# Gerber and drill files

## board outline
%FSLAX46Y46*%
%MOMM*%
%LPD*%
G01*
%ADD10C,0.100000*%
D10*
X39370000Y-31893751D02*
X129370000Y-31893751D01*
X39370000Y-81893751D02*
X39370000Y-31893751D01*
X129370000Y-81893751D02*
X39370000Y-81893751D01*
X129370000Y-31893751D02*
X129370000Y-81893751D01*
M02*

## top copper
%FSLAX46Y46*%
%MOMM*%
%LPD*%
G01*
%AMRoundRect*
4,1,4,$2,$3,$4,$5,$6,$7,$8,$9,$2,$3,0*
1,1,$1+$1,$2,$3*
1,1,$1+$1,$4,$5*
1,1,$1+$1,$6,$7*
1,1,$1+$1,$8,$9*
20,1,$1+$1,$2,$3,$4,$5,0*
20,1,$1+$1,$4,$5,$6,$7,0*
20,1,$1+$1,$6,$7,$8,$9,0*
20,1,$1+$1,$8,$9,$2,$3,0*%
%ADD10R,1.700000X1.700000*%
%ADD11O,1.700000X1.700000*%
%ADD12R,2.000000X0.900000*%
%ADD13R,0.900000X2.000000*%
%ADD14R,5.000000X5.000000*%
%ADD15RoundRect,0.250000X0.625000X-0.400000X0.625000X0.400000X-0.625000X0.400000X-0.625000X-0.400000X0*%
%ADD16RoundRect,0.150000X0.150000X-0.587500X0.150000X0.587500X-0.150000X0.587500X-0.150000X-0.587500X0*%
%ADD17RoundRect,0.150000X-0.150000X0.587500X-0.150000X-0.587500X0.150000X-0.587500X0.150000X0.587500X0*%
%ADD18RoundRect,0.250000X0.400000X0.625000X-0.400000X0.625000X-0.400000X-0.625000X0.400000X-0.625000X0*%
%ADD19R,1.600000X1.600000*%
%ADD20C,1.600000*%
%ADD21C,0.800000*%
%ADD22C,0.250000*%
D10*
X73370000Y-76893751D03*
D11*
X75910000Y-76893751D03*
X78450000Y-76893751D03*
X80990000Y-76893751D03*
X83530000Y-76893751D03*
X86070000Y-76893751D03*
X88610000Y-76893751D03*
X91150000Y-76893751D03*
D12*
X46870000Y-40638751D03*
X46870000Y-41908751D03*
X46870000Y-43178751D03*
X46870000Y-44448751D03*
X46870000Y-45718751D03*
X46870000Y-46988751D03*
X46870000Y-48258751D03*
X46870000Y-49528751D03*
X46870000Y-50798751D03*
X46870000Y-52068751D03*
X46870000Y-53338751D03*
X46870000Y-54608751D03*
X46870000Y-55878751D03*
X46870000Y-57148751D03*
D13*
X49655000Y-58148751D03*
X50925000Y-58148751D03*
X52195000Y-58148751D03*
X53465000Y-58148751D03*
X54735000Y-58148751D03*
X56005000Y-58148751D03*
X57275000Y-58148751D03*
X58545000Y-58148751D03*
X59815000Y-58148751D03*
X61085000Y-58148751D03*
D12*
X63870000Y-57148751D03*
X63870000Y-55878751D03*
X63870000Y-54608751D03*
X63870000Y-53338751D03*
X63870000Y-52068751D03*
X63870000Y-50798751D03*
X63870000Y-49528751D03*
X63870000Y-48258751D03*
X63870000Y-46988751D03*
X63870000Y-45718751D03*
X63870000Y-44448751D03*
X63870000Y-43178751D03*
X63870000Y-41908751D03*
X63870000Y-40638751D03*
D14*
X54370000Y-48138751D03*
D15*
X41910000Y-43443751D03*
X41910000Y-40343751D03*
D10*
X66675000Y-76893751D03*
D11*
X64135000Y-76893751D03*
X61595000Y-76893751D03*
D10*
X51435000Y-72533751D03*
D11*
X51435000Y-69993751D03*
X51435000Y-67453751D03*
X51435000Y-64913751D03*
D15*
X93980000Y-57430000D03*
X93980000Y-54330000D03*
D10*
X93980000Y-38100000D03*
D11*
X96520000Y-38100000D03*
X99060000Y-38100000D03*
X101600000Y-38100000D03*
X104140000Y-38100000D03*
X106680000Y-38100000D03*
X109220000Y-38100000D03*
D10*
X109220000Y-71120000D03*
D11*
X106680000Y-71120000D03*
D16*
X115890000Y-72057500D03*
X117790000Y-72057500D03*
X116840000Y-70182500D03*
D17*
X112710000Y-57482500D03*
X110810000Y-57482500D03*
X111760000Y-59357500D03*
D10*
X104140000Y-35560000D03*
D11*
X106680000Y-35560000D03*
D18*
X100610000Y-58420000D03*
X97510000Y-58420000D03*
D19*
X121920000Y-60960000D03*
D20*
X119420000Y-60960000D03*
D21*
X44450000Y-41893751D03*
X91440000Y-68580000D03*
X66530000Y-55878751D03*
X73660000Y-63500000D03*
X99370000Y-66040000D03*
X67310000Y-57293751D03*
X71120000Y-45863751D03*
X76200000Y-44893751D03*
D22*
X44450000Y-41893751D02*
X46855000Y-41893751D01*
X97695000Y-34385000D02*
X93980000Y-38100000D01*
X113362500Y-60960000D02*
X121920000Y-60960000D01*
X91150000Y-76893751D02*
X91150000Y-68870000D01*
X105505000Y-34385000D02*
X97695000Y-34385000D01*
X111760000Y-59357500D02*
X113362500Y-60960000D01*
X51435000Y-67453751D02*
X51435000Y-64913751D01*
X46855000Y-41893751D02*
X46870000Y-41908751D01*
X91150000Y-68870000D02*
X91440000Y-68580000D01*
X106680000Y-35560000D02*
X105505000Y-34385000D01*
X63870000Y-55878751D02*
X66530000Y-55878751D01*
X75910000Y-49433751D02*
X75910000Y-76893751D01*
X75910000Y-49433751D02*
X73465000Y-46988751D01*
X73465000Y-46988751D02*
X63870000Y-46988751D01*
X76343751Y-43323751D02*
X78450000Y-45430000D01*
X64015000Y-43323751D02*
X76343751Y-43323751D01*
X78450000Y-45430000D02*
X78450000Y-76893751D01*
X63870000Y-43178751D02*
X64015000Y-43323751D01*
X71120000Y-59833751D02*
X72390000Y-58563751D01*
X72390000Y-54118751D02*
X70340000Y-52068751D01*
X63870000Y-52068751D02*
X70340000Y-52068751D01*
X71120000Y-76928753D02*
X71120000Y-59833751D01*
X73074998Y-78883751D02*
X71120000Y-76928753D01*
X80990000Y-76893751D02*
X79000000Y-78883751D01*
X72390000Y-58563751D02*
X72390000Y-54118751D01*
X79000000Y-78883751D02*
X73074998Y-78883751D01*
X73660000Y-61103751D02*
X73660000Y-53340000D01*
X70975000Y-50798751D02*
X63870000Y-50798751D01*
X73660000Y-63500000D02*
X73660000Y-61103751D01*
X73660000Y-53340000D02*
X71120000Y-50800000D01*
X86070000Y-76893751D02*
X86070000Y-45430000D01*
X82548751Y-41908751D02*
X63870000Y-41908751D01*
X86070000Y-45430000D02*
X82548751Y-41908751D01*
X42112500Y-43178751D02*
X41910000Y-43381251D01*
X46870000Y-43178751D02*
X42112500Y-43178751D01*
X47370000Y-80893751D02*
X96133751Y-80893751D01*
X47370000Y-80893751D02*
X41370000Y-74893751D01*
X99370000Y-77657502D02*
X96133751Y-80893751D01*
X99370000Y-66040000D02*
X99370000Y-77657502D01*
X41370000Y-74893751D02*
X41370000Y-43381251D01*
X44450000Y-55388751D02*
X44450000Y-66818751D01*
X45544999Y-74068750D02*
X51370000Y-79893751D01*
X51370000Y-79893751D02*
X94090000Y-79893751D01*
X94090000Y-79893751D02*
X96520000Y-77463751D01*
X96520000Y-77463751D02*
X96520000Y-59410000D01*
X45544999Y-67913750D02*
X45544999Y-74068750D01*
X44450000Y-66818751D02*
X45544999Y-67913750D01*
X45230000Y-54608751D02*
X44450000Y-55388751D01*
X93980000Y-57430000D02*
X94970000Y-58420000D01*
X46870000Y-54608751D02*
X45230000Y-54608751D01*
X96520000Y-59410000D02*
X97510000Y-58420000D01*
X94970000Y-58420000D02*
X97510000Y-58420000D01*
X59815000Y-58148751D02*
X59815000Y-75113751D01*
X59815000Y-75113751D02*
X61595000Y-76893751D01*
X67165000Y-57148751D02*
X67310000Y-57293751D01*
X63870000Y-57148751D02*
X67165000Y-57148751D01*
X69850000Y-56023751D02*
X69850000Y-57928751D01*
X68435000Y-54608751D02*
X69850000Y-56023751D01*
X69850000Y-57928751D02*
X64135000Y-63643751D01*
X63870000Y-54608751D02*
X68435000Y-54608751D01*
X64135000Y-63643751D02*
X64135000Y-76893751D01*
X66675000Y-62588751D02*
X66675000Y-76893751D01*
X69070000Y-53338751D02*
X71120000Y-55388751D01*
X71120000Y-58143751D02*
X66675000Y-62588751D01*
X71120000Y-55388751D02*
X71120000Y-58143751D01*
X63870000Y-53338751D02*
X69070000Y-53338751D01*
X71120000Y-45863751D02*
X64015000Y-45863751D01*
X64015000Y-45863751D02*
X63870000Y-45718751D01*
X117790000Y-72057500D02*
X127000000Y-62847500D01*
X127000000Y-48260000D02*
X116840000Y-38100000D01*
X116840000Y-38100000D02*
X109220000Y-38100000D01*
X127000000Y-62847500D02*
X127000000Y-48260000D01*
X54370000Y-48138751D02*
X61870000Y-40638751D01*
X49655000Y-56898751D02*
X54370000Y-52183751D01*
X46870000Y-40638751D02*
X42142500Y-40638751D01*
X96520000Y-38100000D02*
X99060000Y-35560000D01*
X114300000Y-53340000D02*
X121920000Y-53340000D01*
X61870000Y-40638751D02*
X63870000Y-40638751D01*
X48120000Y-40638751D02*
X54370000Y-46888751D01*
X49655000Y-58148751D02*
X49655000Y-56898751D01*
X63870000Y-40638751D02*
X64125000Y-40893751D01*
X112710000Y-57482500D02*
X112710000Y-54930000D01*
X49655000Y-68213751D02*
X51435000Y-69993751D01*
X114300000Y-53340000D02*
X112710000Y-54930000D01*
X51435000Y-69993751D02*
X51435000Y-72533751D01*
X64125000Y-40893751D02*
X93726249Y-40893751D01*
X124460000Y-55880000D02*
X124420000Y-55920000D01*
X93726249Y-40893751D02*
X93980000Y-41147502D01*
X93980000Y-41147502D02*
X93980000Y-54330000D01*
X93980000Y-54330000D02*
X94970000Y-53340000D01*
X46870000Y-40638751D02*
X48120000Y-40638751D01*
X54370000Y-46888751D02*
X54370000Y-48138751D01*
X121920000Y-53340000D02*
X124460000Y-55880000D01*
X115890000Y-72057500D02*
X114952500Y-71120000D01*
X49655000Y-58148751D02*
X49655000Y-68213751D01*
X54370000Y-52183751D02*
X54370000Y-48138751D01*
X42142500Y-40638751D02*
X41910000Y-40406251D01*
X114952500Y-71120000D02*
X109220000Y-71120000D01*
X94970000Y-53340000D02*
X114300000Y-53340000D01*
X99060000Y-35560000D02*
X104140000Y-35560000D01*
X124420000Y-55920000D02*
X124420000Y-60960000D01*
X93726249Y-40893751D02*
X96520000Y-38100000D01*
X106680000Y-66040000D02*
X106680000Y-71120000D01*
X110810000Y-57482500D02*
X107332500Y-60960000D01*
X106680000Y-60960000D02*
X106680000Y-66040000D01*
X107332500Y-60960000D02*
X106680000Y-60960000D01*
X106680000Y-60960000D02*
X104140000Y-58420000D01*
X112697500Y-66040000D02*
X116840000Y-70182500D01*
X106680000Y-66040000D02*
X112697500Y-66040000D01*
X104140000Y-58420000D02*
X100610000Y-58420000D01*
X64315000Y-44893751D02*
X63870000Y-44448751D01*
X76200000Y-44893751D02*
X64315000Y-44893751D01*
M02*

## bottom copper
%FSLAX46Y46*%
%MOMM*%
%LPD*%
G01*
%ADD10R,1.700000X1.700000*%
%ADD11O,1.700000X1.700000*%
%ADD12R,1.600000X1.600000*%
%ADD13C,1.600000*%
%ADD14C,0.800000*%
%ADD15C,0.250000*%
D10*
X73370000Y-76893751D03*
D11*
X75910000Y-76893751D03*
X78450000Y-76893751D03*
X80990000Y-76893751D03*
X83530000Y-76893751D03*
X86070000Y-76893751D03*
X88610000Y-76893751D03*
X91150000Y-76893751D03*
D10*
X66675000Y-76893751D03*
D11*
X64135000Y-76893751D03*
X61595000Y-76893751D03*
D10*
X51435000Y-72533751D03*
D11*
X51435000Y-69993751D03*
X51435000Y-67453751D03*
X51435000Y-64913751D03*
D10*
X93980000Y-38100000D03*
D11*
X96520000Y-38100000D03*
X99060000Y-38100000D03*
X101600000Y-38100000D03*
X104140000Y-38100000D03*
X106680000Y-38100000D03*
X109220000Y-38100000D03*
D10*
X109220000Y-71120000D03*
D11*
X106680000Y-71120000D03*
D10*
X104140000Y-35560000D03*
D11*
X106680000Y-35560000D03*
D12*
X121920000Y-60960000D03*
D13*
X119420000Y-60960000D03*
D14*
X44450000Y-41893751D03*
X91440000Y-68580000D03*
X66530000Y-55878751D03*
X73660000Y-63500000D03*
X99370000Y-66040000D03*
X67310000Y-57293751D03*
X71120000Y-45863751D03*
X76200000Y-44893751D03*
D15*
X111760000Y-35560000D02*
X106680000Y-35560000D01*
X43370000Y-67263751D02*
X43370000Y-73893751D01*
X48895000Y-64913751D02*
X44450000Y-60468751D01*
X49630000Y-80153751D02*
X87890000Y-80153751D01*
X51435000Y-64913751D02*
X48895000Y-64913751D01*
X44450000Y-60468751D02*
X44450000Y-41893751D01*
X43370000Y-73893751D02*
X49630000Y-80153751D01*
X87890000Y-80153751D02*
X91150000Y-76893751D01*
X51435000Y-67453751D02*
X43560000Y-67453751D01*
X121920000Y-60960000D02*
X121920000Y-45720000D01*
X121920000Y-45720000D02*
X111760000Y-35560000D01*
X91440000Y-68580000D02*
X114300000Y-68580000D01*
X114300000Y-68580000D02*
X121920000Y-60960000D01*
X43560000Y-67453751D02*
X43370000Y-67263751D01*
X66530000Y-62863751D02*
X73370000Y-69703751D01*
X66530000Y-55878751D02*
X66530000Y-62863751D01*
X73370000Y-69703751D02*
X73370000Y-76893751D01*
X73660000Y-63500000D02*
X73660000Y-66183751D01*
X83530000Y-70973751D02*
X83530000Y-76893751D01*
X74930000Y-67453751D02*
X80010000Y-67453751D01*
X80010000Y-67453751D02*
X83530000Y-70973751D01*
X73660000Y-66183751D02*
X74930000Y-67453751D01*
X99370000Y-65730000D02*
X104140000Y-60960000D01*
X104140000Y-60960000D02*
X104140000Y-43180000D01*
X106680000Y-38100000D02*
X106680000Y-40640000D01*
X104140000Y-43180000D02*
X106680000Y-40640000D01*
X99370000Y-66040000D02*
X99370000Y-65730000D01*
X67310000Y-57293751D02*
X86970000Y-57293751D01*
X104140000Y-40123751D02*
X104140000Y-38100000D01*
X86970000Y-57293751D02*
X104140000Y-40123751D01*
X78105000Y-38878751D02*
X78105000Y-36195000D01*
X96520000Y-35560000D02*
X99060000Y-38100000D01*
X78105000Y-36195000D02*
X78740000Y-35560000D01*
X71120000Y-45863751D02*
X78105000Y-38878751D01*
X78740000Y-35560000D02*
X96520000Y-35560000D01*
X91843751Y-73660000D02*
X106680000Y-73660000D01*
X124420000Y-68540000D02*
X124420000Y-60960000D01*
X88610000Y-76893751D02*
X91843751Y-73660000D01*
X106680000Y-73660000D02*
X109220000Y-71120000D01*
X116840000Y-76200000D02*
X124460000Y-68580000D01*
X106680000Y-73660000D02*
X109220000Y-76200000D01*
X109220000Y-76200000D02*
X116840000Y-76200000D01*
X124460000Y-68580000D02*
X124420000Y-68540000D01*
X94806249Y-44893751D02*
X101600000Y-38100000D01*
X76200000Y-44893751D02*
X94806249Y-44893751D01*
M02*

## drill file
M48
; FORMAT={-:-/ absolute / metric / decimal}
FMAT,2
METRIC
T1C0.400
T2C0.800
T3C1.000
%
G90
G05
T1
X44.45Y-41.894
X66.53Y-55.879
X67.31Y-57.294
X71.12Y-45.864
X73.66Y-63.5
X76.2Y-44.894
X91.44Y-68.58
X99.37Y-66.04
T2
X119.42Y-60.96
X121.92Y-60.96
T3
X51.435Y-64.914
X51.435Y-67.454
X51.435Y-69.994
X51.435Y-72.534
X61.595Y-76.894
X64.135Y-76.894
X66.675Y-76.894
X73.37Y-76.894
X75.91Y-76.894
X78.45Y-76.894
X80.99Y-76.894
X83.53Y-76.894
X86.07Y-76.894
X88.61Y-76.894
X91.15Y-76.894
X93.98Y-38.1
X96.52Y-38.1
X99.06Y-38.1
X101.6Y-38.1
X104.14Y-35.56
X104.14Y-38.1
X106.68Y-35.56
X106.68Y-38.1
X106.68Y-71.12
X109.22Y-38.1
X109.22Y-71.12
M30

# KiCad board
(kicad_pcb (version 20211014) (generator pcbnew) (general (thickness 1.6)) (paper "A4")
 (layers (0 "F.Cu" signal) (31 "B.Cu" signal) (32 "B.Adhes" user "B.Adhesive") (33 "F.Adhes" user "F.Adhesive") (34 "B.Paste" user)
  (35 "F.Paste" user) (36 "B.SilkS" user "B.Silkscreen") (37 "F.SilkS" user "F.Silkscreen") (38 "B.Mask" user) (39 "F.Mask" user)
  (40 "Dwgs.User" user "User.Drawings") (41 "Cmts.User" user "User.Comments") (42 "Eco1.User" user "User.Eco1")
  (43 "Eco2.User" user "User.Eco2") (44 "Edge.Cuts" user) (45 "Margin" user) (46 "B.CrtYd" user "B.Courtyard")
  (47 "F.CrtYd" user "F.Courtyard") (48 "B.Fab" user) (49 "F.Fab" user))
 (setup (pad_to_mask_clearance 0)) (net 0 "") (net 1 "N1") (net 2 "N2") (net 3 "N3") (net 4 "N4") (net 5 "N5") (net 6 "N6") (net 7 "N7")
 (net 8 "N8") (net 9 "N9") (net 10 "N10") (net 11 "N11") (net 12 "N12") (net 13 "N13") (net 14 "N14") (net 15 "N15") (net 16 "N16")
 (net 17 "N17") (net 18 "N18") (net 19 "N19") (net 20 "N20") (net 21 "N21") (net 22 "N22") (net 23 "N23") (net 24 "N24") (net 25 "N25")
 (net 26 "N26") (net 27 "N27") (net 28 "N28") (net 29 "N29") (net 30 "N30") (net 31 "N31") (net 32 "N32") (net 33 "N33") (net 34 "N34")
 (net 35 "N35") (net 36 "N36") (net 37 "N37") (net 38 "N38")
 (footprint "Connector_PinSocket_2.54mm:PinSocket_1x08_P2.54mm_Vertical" (layer "F.Cu") (at 73.37 76.893751 90)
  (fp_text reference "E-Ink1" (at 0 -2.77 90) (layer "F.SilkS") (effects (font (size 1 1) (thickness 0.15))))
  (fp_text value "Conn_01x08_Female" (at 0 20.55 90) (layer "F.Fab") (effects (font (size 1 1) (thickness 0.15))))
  (pad "1" thru_hole rect locked (at 0 0 90) (size 1.7 1.7) (drill 1) (layers *.Cu *.Mask) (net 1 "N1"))
  (pad "2" thru_hole oval locked (at 0 2.54 90) (size 1.7 1.7) (drill 1) (layers *.Cu *.Mask) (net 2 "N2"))
  (pad "3" thru_hole oval locked (at 0 5.08 90) (size 1.7 1.7) (drill 1) (layers *.Cu *.Mask) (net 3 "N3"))
  (pad "4" thru_hole oval locked (at 0 7.62 90) (size 1.7 1.7) (drill 1) (layers *.Cu *.Mask) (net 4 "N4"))
  (pad "5" thru_hole oval locked (at 0 10.16 90) (size 1.7 1.7) (drill 1) (layers *.Cu *.Mask) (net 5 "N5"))
  (pad "6" thru_hole oval locked (at 0 12.7 90) (size 1.7 1.7) (drill 1) (layers *.Cu *.Mask) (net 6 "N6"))
  (pad "7" thru_hole oval locked (at 0 15.24 90) (size 1.7 1.7) (drill 1) (layers *.Cu *.Mask) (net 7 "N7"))
  (pad "8" thru_hole oval locked (at 0 17.78 90) (size 1.7 1.7) (drill 1) (layers *.Cu *.Mask) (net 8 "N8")))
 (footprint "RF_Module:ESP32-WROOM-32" (layer "F.Cu") (at 55.37 48.893751)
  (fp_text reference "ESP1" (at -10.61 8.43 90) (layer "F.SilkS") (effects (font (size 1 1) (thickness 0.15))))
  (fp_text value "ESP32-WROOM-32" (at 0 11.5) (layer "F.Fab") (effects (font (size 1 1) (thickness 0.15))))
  (pad "1" smd rect locked (at -8.5 -8.255) (size 2 0.9) (layers "F.Cu" "F.Paste" "F.Mask") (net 7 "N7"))
  (pad "2" smd rect locked (at -8.5 -6.985) (size 2 0.9) (layers "F.Cu" "F.Paste" "F.Mask") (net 8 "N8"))
  (pad "3" smd rect locked (at -8.5 -5.715) (size 2 0.9) (layers "F.Cu" "F.Paste" "F.Mask") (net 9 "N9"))
  (pad "4" smd rect locked (at -8.5 -4.445) (size 2 0.9) (layers "F.Cu" "F.Paste" "F.Mask") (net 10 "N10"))
  (pad "5" smd rect locked (at -8.5 -3.175) (size 2 0.9) (layers "F.Cu" "F.Paste" "F.Mask") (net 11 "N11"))
  (pad "6" smd rect locked (at -8.5 -1.905) (size 2 0.9) (layers "F.Cu" "F.Paste" "F.Mask") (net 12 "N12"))
  (pad "7" smd rect locked (at -8.5 -0.635) (size 2 0.9) (layers "F.Cu" "F.Paste" "F.Mask") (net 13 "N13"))
  (pad "8" smd rect locked (at -8.5 0.635) (size 2 0.9) (layers "F.Cu" "F.Paste" "F.Mask") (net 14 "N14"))
  (pad "9" smd rect locked (at -8.5 1.905) (size 2 0.9) (layers "F.Cu" "F.Paste" "F.Mask") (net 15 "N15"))
  (pad "10" smd rect locked (at -8.5 3.175) (size 2 0.9) (layers "F.Cu" "F.Paste" "F.Mask") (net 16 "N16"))
  (pad "11" smd rect locked (at -8.5 4.445) (size 2 0.9) (layers "F.Cu" "F.Paste" "F.Mask") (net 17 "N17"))
  (pad "12" smd rect locked (at -8.5 5.715) (size 2 0.9) (layers "F.Cu" "F.Paste" "F.Mask") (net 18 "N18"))
  (pad "13" smd rect locked (at -8.5 6.985) (size 2 0.9) (layers "F.Cu" "F.Paste" "F.Mask") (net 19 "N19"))
  (pad "14" smd rect locked (at -8.5 8.255) (size 2 0.9) (layers "F.Cu" "F.Paste" "F.Mask") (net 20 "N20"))
  (pad "15" smd rect locked (at -5.715 9.255 90) (size 2 0.9) (layers "F.Cu" "F.Paste" "F.Mask") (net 7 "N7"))
  (pad "16" smd rect locked (at -4.445 9.255 90) (size 2 0.9) (layers "F.Cu" "F.Paste" "F.Mask") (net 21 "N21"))
  (pad "17" smd rect locked (at -3.175 9.255 90) (size 2 0.9) (layers "F.Cu" "F.Paste" "F.Mask") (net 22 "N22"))
  (pad "18" smd rect locked (at -1.905 9.255 90) (size 2 0.9) (layers "F.Cu" "F.Paste" "F.Mask") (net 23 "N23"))
  (pad "19" smd rect locked (at -0.635 9.255 90) (size 2 0.9) (layers "F.Cu" "F.Paste" "F.Mask") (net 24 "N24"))
  (pad "20" smd rect locked (at 0.635 9.255 90) (size 2 0.9) (layers "F.Cu" "F.Paste" "F.Mask") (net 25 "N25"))
  (pad "21" smd rect locked (at 1.905 9.255 90) (size 2 0.9) (layers "F.Cu" "F.Paste" "F.Mask") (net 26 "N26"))
  (pad "22" smd rect locked (at 3.175 9.255 90) (size 2 0.9) (layers "F.Cu" "F.Paste" "F.Mask") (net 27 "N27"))
  (pad "23" smd rect locked (at 4.445 9.255 90) (size 2 0.9) (layers "F.Cu" "F.Paste" "F.Mask") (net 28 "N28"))
  (pad "24" smd rect locked (at 5.715 9.255 90) (size 2 0.9) (layers "F.Cu" "F.Paste" "F.Mask") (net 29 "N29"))
  (pad "25" smd rect locked (at 8.5 8.255) (size 2 0.9) (layers "F.Cu" "F.Paste" "F.Mask") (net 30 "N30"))
  (pad "26" smd rect locked (at 8.5 6.985) (size 2 0.9) (layers "F.Cu" "F.Paste" "F.Mask") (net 1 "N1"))
  (pad "27" smd rect locked (at 8.5 5.715) (size 2 0.9) (layers "F.Cu" "F.Paste" "F.Mask") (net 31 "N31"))
  (pad "28" smd rect locked (at 8.5 4.445) (size 2 0.9) (layers "F.Cu" "F.Paste" "F.Mask") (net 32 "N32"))
  (pad "29" smd rect locked (at 8.5 3.175) (size 2 0.9) (layers "F.Cu" "F.Paste" "F.Mask") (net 4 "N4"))
  (pad "30" smd rect locked (at 8.5 1.905) (size 2 0.9) (layers "F.Cu" "F.Paste" "F.Mask") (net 5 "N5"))
  (pad "31" smd rect locked (at 8.5 0.635) (size 2 0.9) (layers "F.Cu" "F.Paste" "F.Mask") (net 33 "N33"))
  (pad "32" smd rect locked (at 8.5 -0.635) (size 2 0.9) (layers "F.Cu" "F.Paste" "F.Mask") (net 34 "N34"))
  (pad "33" smd rect locked (at 8.5 -1.905) (size 2 0.9) (layers "F.Cu" "F.Paste" "F.Mask") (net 2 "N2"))
  (pad "34" smd rect locked (at 8.5 -3.175) (size 2 0.9) (layers "F.Cu" "F.Paste" "F.Mask") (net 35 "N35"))
  (pad "35" smd rect locked (at 8.5 -4.445) (size 2 0.9) (layers "F.Cu" "F.Paste" "F.Mask") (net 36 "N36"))
  (pad "36" smd rect locked (at 8.5 -5.715) (size 2 0.9) (layers "F.Cu" "F.Paste" "F.Mask") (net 3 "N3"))
  (pad "37" smd rect locked (at 8.5 -6.985) (size 2 0.9) (layers "F.Cu" "F.Paste" "F.Mask") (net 6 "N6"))
  (pad "38" smd rect locked (at 8.5 -8.255) (size 2 0.9) (layers "F.Cu" "F.Paste" "F.Mask") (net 7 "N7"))
  (pad "39" smd rect locked (at -1 -0.755) (size 5 5) (layers "F.Cu" "F.Paste" "F.Mask") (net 7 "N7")))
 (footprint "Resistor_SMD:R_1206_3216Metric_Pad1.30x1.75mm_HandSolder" (layer "F.Cu") (at 41.91 41.893751 90)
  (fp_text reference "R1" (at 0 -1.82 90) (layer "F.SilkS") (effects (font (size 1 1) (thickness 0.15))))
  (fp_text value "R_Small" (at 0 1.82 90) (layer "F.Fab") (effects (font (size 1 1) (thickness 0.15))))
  (pad "1" smd roundrect (at -1.55 0 90) (size 1.3 1.75) (layers "F.Cu" "F.Paste" "F.Mask") (roundrect_rratio 0.192308) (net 9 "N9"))
  (pad "2" smd roundrect (at 1.55 0 90) (size 1.3 1.75) (layers "F.Cu" "F.Paste" "F.Mask") (roundrect_rratio 0.192308) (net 7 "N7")))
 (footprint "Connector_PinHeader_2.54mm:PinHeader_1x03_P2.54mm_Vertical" (layer "F.Cu") (at 66.675 76.893751 -90)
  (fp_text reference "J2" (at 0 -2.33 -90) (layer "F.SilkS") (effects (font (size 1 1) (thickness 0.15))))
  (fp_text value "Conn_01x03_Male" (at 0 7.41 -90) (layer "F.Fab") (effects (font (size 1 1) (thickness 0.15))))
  (pad "1" thru_hole rect (at 0 0 270) (size 1.7 1.7) (drill 1) (layers *.Cu *.Mask) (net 32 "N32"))
  (pad "2" thru_hole oval (at 0 2.54 270) (size 1.7 1.7) (drill 1) (layers *.Cu *.Mask) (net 31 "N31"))
  (pad "3" thru_hole oval (at 0 5.08 270) (size 1.7 1.7) (drill 1) (layers *.Cu *.Mask) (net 28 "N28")))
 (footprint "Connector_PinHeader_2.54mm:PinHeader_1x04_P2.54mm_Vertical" (layer "F.Cu") (at 51.435 72.533751 180)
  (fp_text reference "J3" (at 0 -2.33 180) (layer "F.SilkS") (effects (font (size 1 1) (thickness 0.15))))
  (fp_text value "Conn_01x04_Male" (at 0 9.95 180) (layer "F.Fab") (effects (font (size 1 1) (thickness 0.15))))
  (pad "1" thru_hole rect (at 0 0 180) (size 1.7 1.7) (drill 1) (layers *.Cu *.Mask) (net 7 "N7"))
  (pad "2" thru_hole oval (at 0 2.54 180) (size 1.7 1.7) (drill 1) (layers *.Cu *.Mask) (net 7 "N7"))
  (pad "3" thru_hole oval (at 0 5.08 180) (size 1.7 1.7) (drill 1) (layers *.Cu *.Mask) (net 8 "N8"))
  (pad "4" thru_hole oval (at 0 7.62 180) (size 1.7 1.7) (drill 1) (layers *.Cu *.Mask) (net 8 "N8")))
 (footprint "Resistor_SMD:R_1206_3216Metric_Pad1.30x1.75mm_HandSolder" (layer "F.Cu") (at 93.98 55.88 90)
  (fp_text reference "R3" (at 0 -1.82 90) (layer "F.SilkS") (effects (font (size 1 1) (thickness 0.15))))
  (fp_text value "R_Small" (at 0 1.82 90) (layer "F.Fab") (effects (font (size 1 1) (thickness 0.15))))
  (pad "1" smd roundrect (at -1.55 0 90) (size 1.3 1.75) (layers "F.Cu" "F.Paste" "F.Mask") (roundrect_rratio 0.192308) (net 18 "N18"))
  (pad "2" smd roundrect (at 1.55 0 90) (size 1.3 1.75) (layers "F.Cu" "F.Paste" "F.Mask") (roundrect_rratio 0.192308) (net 7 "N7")))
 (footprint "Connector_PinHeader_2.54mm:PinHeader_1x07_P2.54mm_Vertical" (layer "F.Cu") (at 93.98 38.1 90)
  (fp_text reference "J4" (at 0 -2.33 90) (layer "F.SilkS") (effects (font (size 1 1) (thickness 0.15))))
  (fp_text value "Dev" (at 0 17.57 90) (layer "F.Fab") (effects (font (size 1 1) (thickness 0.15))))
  (pad "1" thru_hole rect (at 0 0 90) (size 1.7 1.7) (drill 1) (layers *.Cu *.Mask) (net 8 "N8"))
  (pad "2" thru_hole oval (at 0 2.54 90) (size 1.7 1.7) (drill 1) (layers *.Cu *.Mask) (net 7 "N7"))
  (pad "3" thru_hole oval (at 0 5.08 90) (size 1.7 1.7) (drill 1) (layers *.Cu *.Mask) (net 35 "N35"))
  (pad "4" thru_hole oval (at 0 7.62 90) (size 1.7 1.7) (drill 1) (layers *.Cu *.Mask) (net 36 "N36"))
  (pad "5" thru_hole oval (at 0 10.16 90) (size 1.7 1.7) (drill 1) (layers *.Cu *.Mask) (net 30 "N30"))
  (pad "6" thru_hole oval (at 0 12.7 90) (size 1.7 1.7) (drill 1) (layers *.Cu *.Mask) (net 9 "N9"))
  (pad "7" thru_hole oval (at 0 15.24 90) (size 1.7 1.7) (drill 1) (layers *.Cu *.Mask) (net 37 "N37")))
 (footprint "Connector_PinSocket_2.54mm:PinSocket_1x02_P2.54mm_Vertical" (layer "F.Cu") (at 109.22 71.12 -90)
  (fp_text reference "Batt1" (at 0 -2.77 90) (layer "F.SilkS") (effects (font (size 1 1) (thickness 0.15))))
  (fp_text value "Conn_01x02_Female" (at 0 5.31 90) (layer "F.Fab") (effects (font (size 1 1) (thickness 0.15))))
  (pad "1" thru_hole rect (at 0 0 270) (size 1.7 1.7) (drill 1) (layers *.Cu *.Mask) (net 7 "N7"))
  (pad "2" thru_hole oval (at 0 2.54 270) (size 1.7 1.7) (drill 1) (layers *.Cu *.Mask) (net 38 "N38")))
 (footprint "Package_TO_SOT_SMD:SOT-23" (layer "F.Cu") (at 116.84 71.12 90)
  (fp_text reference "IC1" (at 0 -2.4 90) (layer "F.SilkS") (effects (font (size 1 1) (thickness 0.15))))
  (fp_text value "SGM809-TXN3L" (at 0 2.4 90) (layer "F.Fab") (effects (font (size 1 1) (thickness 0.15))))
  (pad "1" smd roundrect (at -0.9375 -0.95 90) (size 1.475 0.6) (layers "F.Cu" "F.Paste" "F.Mask") (roundrect_rratio 0.25) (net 7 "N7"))
  (pad "2" smd roundrect (at -0.9375 0.95 90) (size 1.475 0.6) (layers "F.Cu" "F.Paste" "F.Mask") (roundrect_rratio 0.25) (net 37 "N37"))
  (pad "3" smd roundrect (at 0.9375 0 90) (size 1.475 0.6) (layers "F.Cu" "F.Paste" "F.Mask") (roundrect_rratio 0.25) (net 38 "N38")))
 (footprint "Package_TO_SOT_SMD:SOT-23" (layer "F.Cu") (at 111.76 58.42 -90)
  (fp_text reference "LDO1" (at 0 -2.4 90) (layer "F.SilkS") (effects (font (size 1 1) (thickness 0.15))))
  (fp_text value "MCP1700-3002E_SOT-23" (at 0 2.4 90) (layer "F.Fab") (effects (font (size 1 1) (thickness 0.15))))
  (pad "1" smd roundrect (at -0.9375 -0.95 270) (size 1.475 0.6) (layers "F.Cu" "F.Paste" "F.Mask") (roundrect_rratio 0.25) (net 7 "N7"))
  (pad "2" smd roundrect (at -0.9375 0.95 270) (size 1.475 0.6) (layers "F.Cu" "F.Paste" "F.Mask") (roundrect_rratio 0.25) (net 38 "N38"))
  (pad "3" smd roundrect (at 0.9375 0 270) (size 1.475 0.6) (layers "F.Cu" "F.Paste" "F.Mask") (roundrect_rratio 0.25) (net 8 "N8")))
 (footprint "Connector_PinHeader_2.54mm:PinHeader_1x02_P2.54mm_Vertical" (layer "F.Cu") (at 104.14 35.56 90)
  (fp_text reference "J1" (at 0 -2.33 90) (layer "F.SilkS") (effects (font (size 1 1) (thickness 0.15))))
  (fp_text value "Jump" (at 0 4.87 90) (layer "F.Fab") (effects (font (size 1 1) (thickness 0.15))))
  (pad "1" thru_hole rect (at 0 0 90) (size 1.7 1.7) (drill 1) (layers *.Cu *.Mask) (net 7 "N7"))
  (pad "2" thru_hole oval (at 0 2.54 90) (size 1.7 1.7) (drill 1) (layers *.Cu *.Mask) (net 8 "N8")))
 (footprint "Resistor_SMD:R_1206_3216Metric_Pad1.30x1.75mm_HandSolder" (layer "F.Cu") (at 99.06 58.42 180)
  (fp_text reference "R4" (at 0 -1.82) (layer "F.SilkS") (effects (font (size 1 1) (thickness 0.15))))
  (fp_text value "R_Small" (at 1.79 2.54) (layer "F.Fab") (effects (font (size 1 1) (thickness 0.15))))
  (pad "1" smd roundrect (at -1.55 0 180) (size 1.3 1.75) (layers "F.Cu" "F.Paste" "F.Mask") (roundrect_rratio 0.192308) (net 38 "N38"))
  (pad "2" smd roundrect (at 1.55 0 180) (size 1.3 1.75) (layers "F.Cu" "F.Paste" "F.Mask") (roundrect_rratio 0.192308) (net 18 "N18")))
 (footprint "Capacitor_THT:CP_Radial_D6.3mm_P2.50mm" (layer "B.Cu") (at 121.92 60.96 180)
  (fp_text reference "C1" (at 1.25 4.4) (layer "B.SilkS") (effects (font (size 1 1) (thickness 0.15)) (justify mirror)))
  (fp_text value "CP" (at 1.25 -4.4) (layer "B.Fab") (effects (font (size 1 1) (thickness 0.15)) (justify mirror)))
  (pad "1" thru_hole rect (at 0 0 180) (size 1.6 1.6) (drill 0.8) (layers *.Cu *.Mask) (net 8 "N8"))
  (pad "2" thru_hole circle (at 2.5 0 180) (size 1.6 1.6) (drill 0.8) (layers *.Cu *.Mask) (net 7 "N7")))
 (gr_line (start 39.37 31.893751) (end 129.37 31.893751) (layer "Edge.Cuts") (width 0.1))
 (gr_line (start 39.37 81.893751) (end 39.37 31.893751) (layer "Edge.Cuts") (width 0.1))
 (gr_line (start 129.37 81.893751) (end 39.37 81.893751) (layer "Edge.Cuts") (width 0.1))
 (gr_line (start 129.37 31.893751) (end 129.37 81.893751) (layer "Edge.Cuts") (width 0.1))
 (segment (start 44.45 41.893751) (end 46.855 41.893751) (width 0.25) (layer "F.Cu") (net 8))
 (segment (start 97.695 34.385) (end 93.98 38.1) (width 0.25) (layer "F.Cu") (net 8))
 (segment (start 113.3625 60.96) (end 121.92 60.96) (width 0.25) (layer "F.Cu") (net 8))
 (segment (start 91.15 76.893751) (end 91.15 68.87) (width 0.25) (layer "F.Cu") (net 8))
 (segment (start 105.505 34.385) (end 97.695 34.385) (width 0.25) (layer "F.Cu") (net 8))
 (segment (start 111.76 59.3575) (end 113.3625 60.96) (width 0.25) (layer "F.Cu") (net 8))
 (segment (start 51.435 67.453751) (end 51.435 64.913751) (width 0.25) (layer "F.Cu") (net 8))
 (segment (start 46.855 41.893751) (end 46.87 41.908751) (width 0.25) (layer "F.Cu") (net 8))
 (segment (start 91.15 68.87) (end 91.44 68.58) (width 0.25) (layer "F.Cu") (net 8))
 (segment (start 106.68 35.56) (end 105.505 34.385) (width 0.25) (layer "F.Cu") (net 8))
 (via (at 44.45 41.893751) (size 0.8) (drill 0.4) (layers "F.Cu" "B.Cu") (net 8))
 (via (at 91.44 68.58) (size 0.8) (drill 0.4) (layers "F.Cu" "B.Cu") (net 8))
 (segment (start 111.76 35.56) (end 106.68 35.56) (width 0.25) (layer "B.Cu") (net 8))
 (segment (start 43.37 67.263751) (end 43.37 73.893751) (width 0.25) (layer "B.Cu") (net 8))
 (segment (start 48.895 64.913751) (end 44.45 60.468751) (width 0.25) (layer "B.Cu") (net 8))
 (segment (start 49.63 80.153751) (end 87.89 80.153751) (width 0.25) (layer "B.Cu") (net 8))
 (segment (start 51.435 64.913751) (end 48.895 64.913751) (width 0.25) (layer "B.Cu") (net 8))
 (segment (start 44.45 60.468751) (end 44.45 41.893751) (width 0.25) (layer "B.Cu") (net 8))
 (segment (start 43.37 73.893751) (end 49.63 80.153751) (width 0.25) (layer "B.Cu") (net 8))
 (segment (start 87.89 80.153751) (end 91.15 76.893751) (width 0.25) (layer "B.Cu") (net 8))
 (segment (start 51.435 67.453751) (end 43.56 67.453751) (width 0.25) (layer "B.Cu") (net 8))
 (segment (start 121.92 60.96) (end 121.92 45.72) (width 0.25) (layer "B.Cu") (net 8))
 (segment (start 121.92 45.72) (end 111.76 35.56) (width 0.25) (layer "B.Cu") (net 8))
 (segment (start 91.44 68.58) (end 114.3 68.58) (width 0.25) (layer "B.Cu") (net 8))
 (segment (start 114.3 68.58) (end 121.92 60.96) (width 0.25) (layer "B.Cu") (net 8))
 (segment (start 43.56 67.453751) (end 43.37 67.263751) (width 0.25) (layer "B.Cu") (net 8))
 (segment (start 63.87 55.878751) (end 66.53 55.878751) (width 0.25) (layer "F.Cu") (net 1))
 (via (at 66.53 55.878751) (size 0.8) (drill 0.4) (layers "F.Cu" "B.Cu") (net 1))
 (segment (start 66.53 62.863751) (end 73.37 69.703751) (width 0.25) (layer "B.Cu") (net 1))
 (segment (start 66.53 55.878751) (end 66.53 62.863751) (width 0.25) (layer "B.Cu") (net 1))
 (segment (start 73.37 69.703751) (end 73.37 76.893751) (width 0.25) (layer "B.Cu") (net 1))
 (segment (start 75.91 49.433751) (end 75.91 76.893751) (width 0.25) (layer "F.Cu") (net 2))
 (segment (start 75.91 49.433751) (end 73.465 46.988751) (width 0.25) (layer "F.Cu") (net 2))
 (segment (start 73.465 46.988751) (end 63.87 46.988751) (width 0.25) (layer "F.Cu") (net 2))
 (segment (start 76.343751 43.323751) (end 78.45 45.43) (width 0.25) (layer "F.Cu") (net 3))
 (segment (start 64.015 43.323751) (end 76.343751 43.323751) (width 0.25) (layer "F.Cu") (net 3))
 (segment (start 78.45 45.43) (end 78.45 76.893751) (width 0.25) (layer "F.Cu") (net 3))
 (segment (start 63.87 43.178751) (end 64.015 43.323751) (width 0.25) (layer "F.Cu") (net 3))
 (segment (start 71.12 59.833751) (end 72.39 58.563751) (width 0.25) (layer "F.Cu") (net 4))
 (segment (start 72.39 54.118751) (end 70.34 52.068751) (width 0.25) (layer "F.Cu") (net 4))
 (segment (start 63.87 52.068751) (end 70.34 52.068751) (width 0.25) (layer "F.Cu") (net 4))
 (segment (start 71.12 76.928753) (end 71.12 59.833751) (width 0.25) (layer "F.Cu") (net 4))
 (segment (start 73.074998 78.883751) (end 71.12 76.928753) (width 0.25) (layer "F.Cu") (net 4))
 (segment (start 80.99 76.893751) (end 79 78.883751) (width 0.25) (layer "F.Cu") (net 4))
 (segment (start 72.39 58.563751) (end 72.39 54.118751) (width 0.25) (layer "F.Cu") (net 4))
 (segment (start 79 78.883751) (end 73.074998 78.883751) (width 0.25) (layer "F.Cu") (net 4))
 (segment (start 73.66 61.103751) (end 73.66 53.34) (width 0.25) (layer "F.Cu") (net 5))
 (segment (start 70.975 50.798751) (end 63.87 50.798751) (width 0.25) (layer "F.Cu") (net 5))
 (segment (start 73.66 63.5) (end 73.66 61.103751) (width 0.25) (layer "F.Cu") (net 5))
 (segment (start 73.66 53.34) (end 71.12 50.8) (width 0.25) (layer "F.Cu") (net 5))
 (via (at 73.66 63.5) (size 0.8) (drill 0.4) (layers "F.Cu" "B.Cu") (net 5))
 (segment (start 73.66 63.5) (end 73.66 66.183751) (width 0.25) (layer "B.Cu") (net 5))
 (segment (start 83.53 70.973751) (end 83.53 76.893751) (width 0.25) (layer "B.Cu") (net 5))
 (segment (start 74.93 67.453751) (end 80.01 67.453751) (width 0.25) (layer "B.Cu") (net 5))
 (segment (start 80.01 67.453751) (end 83.53 70.973751) (width 0.25) (layer "B.Cu") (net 5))
 (segment (start 73.66 66.183751) (end 74.93 67.453751) (width 0.25) (layer "B.Cu") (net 5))
 (segment (start 86.07 76.893751) (end 86.07 45.43) (width 0.25) (layer "F.Cu") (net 6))
 (segment (start 82.548751 41.908751) (end 63.87 41.908751) (width 0.25) (layer "F.Cu") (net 6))
 (segment (start 86.07 45.43) (end 82.548751 41.908751) (width 0.25) (layer "F.Cu") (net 6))
 (segment (start 42.1125 43.178751) (end 41.91 43.381251) (width 0.25) (layer "F.Cu") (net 9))
 (segment (start 46.87 43.178751) (end 42.1125 43.178751) (width 0.25) (layer "F.Cu") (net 9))
 (segment (start 47.37 80.893751) (end 96.133751 80.893751) (width 0.25) (layer "F.Cu") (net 9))
 (segment (start 47.37 80.893751) (end 41.37 74.893751) (width 0.25) (layer "F.Cu") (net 9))
 (segment (start 99.37 77.657502) (end 96.133751 80.893751) (width 0.25) (layer "F.Cu") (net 9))
 (segment (start 99.37 66.04) (end 99.37 77.657502) (width 0.25) (layer "F.Cu") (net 9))
 (segment (start 41.37 74.893751) (end 41.37 43.381251) (width 0.25) (layer "F.Cu") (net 9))
 (via (at 99.37 66.04) (size 0.8) (drill 0.4) (layers "F.Cu" "B.Cu") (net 9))
 (segment (start 99.37 65.73) (end 104.14 60.96) (width 0.25) (layer "B.Cu") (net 9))
 (segment (start 104.14 60.96) (end 104.14 43.18) (width 0.25) (layer "B.Cu") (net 9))
 (segment (start 106.68 38.1) (end 106.68 40.64) (width 0.25) (layer "B.Cu") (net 9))
 (segment (start 104.14 43.18) (end 106.68 40.64) (width 0.25) (layer "B.Cu") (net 9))
 (segment (start 99.37 66.04) (end 99.37 65.73) (width 0.25) (layer "B.Cu") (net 9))
 (segment (start 44.45 55.388751) (end 44.45 66.818751) (width 0.25) (layer "F.Cu") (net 18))
 (segment (start 45.544999 74.06875) (end 51.37 79.893751) (width 0.25) (layer "F.Cu") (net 18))
 (segment (start 51.37 79.893751) (end 94.09 79.893751) (width 0.25) (layer "F.Cu") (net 18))
 (segment (start 94.09 79.893751) (end 96.52 77.463751) (width 0.25) (layer "F.Cu") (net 18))
 (segment (start 96.52 77.463751) (end 96.52 59.41) (width 0.25) (layer "F.Cu") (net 18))
 (segment (start 45.544999 67.91375) (end 45.544999 74.06875) (width 0.25) (layer "F.Cu") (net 18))
 (segment (start 44.45 66.818751) (end 45.544999 67.91375) (width 0.25) (layer "F.Cu") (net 18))
 (segment (start 45.23 54.608751) (end 44.45 55.388751) (width 0.25) (layer "F.Cu") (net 18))
 (segment (start 93.98 57.43) (end 94.97 58.42) (width 0.25) (layer "F.Cu") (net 18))
 (segment (start 46.87 54.608751) (end 45.23 54.608751) (width 0.25) (layer "F.Cu") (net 18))
 (segment (start 96.52 59.41) (end 97.51 58.42) (width 0.25) (layer "F.Cu") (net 18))
 (segment (start 94.97 58.42) (end 97.51 58.42) (width 0.25) (layer "F.Cu") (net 18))
 (segment (start 59.815 58.148751) (end 59.815 75.113751) (width 0.25) (layer "F.Cu") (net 28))
 (segment (start 59.815 75.113751) (end 61.595 76.893751) (width 0.25) (layer "F.Cu") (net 28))
 (segment (start 67.165 57.148751) (end 67.31 57.293751) (width 0.25) (layer "F.Cu") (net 30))
 (segment (start 63.87 57.148751) (end 67.165 57.148751) (width 0.25) (layer "F.Cu") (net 30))
 (via (at 67.31 57.293751) (size 0.8) (drill 0.4) (layers "F.Cu" "B.Cu") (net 30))
 (segment (start 67.31 57.293751) (end 86.97 57.293751) (width 0.25) (layer "B.Cu") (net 30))
 (segment (start 104.14 40.123751) (end 104.14 38.1) (width 0.25) (layer "B.Cu") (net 30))
 (segment (start 86.97 57.293751) (end 104.14 40.123751) (width 0.25) (layer "B.Cu") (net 30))
 (segment (start 69.85 56.023751) (end 69.85 57.928751) (width 0.25) (layer "F.Cu") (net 31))
 (segment (start 68.435 54.608751) (end 69.85 56.023751) (width 0.25) (layer "F.Cu") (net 31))
 (segment (start 69.85 57.928751) (end 64.135 63.643751) (width 0.25) (layer "F.Cu") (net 31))
 (segment (start 63.87 54.608751) (end 68.435 54.608751) (width 0.25) (layer "F.Cu") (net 31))
 (segment (start 64.135 63.643751) (end 64.135 76.893751) (width 0.25) (layer "F.Cu") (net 31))
 (segment (start 66.675 62.588751) (end 66.675 76.893751) (width 0.25) (layer "F.Cu") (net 32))
 (segment (start 69.07 53.338751) (end 71.12 55.388751) (width 0.25) (layer "F.Cu") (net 32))
 (segment (start 71.12 58.143751) (end 66.675 62.588751) (width 0.25) (layer "F.Cu") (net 32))
 (segment (start 71.12 55.388751) (end 71.12 58.143751) (width 0.25) (layer "F.Cu") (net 32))
 (segment (start 63.87 53.338751) (end 69.07 53.338751) (width 0.25) (layer "F.Cu") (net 32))
 (segment (start 71.12 45.863751) (end 64.015 45.863751) (width 0.25) (layer "F.Cu") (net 35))
 (segment (start 64.015 45.863751) (end 63.87 45.718751) (width 0.25) (layer "F.Cu") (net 35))
 (via (at 71.12 45.863751) (size 0.8) (drill 0.4) (layers "F.Cu" "B.Cu") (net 35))
 (segment (start 78.105 38.878751) (end 78.105 36.195) (width 0.25) (layer "B.Cu") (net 35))
 (segment (start 96.52 35.56) (end 99.06 38.1) (width 0.25) (layer "B.Cu") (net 35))
 (segment (start 78.105 36.195) (end 78.74 35.56) (width 0.25) (layer "B.Cu") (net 35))
 (segment (start 71.12 45.863751) (end 78.105 38.878751) (width 0.25) (layer "B.Cu") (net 35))
 (segment (start 78.74 35.56) (end 96.52 35.56) (width 0.25) (layer "B.Cu") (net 35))
 (segment (start 117.79 72.0575) (end 127 62.8475) (width 0.25) (layer "F.Cu") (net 37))
 (segment (start 127 48.26) (end 116.84 38.1) (width 0.25) (layer "F.Cu") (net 37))
 (segment (start 116.84 38.1) (end 109.22 38.1) (width 0.25) (layer "F.Cu") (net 37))
 (segment (start 127 62.8475) (end 127 48.26) (width 0.25) (layer "F.Cu") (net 37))
 (segment (start 54.37 48.138751) (end 61.87 40.638751) (width 0.25) (layer "F.Cu") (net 7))
 (segment (start 49.655 56.898751) (end 54.37 52.183751) (width 0.25) (layer "F.Cu") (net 7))
 (segment (start 46.87 40.638751) (end 42.1425 40.638751) (width 0.25) (layer "F.Cu") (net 7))
 (segment (start 96.52 38.1) (end 99.06 35.56) (width 0.25) (layer "F.Cu") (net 7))
 (segment (start 114.3 53.34) (end 121.92 53.34) (width 0.25) (layer "F.Cu") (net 7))
 (segment (start 61.87 40.638751) (end 63.87 40.638751) (width 0.25) (layer "F.Cu") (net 7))
 (segment (start 48.12 40.638751) (end 54.37 46.888751) (width 0.25) (layer "F.Cu") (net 7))
 (segment (start 49.655 58.148751) (end 49.655 56.898751) (width 0.25) (layer "F.Cu") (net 7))
 (segment (start 63.87 40.638751) (end 64.125 40.893751) (width 0.25) (layer "F.Cu") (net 7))
 (segment (start 112.71 57.4825) (end 112.71 54.93) (width 0.25) (layer "F.Cu") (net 7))
 (segment (start 49.655 68.213751) (end 51.435 69.993751) (width 0.25) (layer "F.Cu") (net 7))
 (segment (start 114.3 53.34) (end 112.71 54.93) (width 0.25) (layer "F.Cu") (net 7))
 (segment (start 51.435 69.993751) (end 51.435 72.533751) (width 0.25) (layer "F.Cu") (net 7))
 (segment (start 64.125 40.893751) (end 93.726249 40.893751) (width 0.25) (layer "F.Cu") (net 7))
 (segment (start 124.46 55.88) (end 124.42 55.92) (width 0.25) (layer "F.Cu") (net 7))
 (segment (start 93.726249 40.893751) (end 93.98 41.147502) (width 0.25) (layer "F.Cu") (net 7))
 (segment (start 93.98 41.147502) (end 93.98 54.33) (width 0.25) (layer "F.Cu") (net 7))
 (segment (start 93.98 54.33) (end 94.97 53.34) (width 0.25) (layer "F.Cu") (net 7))
 (segment (start 46.87 40.638751) (end 48.12 40.638751) (width 0.25) (layer "F.Cu") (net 7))
 (segment (start 54.37 46.888751) (end 54.37 48.138751) (width 0.25) (layer "F.Cu") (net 7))
 (segment (start 121.92 53.34) (end 124.46 55.88) (width 0.25) (layer "F.Cu") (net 7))
 (segment (start 115.89 72.0575) (end 114.9525 71.12) (width 0.25) (layer "F.Cu") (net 7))
 (segment (start 49.655 58.148751) (end 49.655 68.213751) (width 0.25) (layer "F.Cu") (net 7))
 (segment (start 54.37 52.183751) (end 54.37 48.138751) (width 0.25) (layer "F.Cu") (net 7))
 (segment (start 42.1425 40.638751) (end 41.91 40.406251) (width 0.25) (layer "F.Cu") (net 7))
 (segment (start 114.9525 71.12) (end 109.22 71.12) (width 0.25) (layer "F.Cu") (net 7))
 (segment (start 94.97 53.34) (end 114.3 53.34) (width 0.25) (layer "F.Cu") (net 7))
 (segment (start 99.06 35.56) (end 104.14 35.56) (width 0.25) (layer "F.Cu") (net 7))
 (segment (start 124.42 55.92) (end 124.42 60.96) (width 0.25) (layer "F.Cu") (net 7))
 (segment (start 93.726249 40.893751) (end 96.52 38.1) (width 0.25) (layer "F.Cu") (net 7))
 (segment (start 91.843751 73.66) (end 106.68 73.66) (width 0.25) (layer "B.Cu") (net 7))
 (segment (start 124.42 68.54) (end 124.42 60.96) (width 0.25) (layer "B.Cu") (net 7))
 (segment (start 88.61 76.893751) (end 91.843751 73.66) (width 0.25) (layer "B.Cu") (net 7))
 (segment (start 106.68 73.66) (end 109.22 71.12) (width 0.25) (layer "B.Cu") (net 7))
 (segment (start 116.84 76.2) (end 124.46 68.58) (width 0.25) (layer "B.Cu") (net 7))
 (segment (start 106.68 73.66) (end 109.22 76.2) (width 0.25) (layer "B.Cu") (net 7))
 (segment (start 109.22 76.2) (end 116.84 76.2) (width 0.25) (layer "B.Cu") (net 7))
 (segment (start 124.46 68.58) (end 124.42 68.54) (width 0.25) (layer "B.Cu") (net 7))
 (segment (start 106.68 66.04) (end 106.68 71.12) (width 0.25) (layer "F.Cu") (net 38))
 (segment (start 110.81 57.4825) (end 107.3325 60.96) (width 0.25) (layer "F.Cu") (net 38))
 (segment (start 106.68 60.96) (end 106.68 66.04) (width 0.25) (layer "F.Cu") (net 38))
 (segment (start 107.3325 60.96) (end 106.68 60.96) (width 0.25) (layer "F.Cu") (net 38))
 (segment (start 106.68 60.96) (end 104.14 58.42) (width 0.25) (layer "F.Cu") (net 38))
 (segment (start 112.6975 66.04) (end 116.84 70.1825) (width 0.25) (layer "F.Cu") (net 38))
 (segment (start 106.68 66.04) (end 112.6975 66.04) (width 0.25) (layer "F.Cu") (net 38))
 (segment (start 104.14 58.42) (end 100.61 58.42) (width 0.25) (layer "F.Cu") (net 38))
 (segment (start 64.315 44.893751) (end 63.87 44.448751) (width 0.25) (layer "F.Cu") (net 36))
 (segment (start 76.2 44.893751) (end 64.315 44.893751) (width 0.25) (layer "F.Cu") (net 36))
 (via (at 76.2 44.893751) (size 0.8) (drill 0.4) (layers "F.Cu" "B.Cu") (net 36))
 (segment (start 94.806249 44.893751) (end 101.6 38.1) (width 0.25) (layer "B.Cu") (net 36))
 (segment (start 76.2 44.893751) (end 94.806249 44.893751) (width 0.25) (layer "B.Cu") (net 36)))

